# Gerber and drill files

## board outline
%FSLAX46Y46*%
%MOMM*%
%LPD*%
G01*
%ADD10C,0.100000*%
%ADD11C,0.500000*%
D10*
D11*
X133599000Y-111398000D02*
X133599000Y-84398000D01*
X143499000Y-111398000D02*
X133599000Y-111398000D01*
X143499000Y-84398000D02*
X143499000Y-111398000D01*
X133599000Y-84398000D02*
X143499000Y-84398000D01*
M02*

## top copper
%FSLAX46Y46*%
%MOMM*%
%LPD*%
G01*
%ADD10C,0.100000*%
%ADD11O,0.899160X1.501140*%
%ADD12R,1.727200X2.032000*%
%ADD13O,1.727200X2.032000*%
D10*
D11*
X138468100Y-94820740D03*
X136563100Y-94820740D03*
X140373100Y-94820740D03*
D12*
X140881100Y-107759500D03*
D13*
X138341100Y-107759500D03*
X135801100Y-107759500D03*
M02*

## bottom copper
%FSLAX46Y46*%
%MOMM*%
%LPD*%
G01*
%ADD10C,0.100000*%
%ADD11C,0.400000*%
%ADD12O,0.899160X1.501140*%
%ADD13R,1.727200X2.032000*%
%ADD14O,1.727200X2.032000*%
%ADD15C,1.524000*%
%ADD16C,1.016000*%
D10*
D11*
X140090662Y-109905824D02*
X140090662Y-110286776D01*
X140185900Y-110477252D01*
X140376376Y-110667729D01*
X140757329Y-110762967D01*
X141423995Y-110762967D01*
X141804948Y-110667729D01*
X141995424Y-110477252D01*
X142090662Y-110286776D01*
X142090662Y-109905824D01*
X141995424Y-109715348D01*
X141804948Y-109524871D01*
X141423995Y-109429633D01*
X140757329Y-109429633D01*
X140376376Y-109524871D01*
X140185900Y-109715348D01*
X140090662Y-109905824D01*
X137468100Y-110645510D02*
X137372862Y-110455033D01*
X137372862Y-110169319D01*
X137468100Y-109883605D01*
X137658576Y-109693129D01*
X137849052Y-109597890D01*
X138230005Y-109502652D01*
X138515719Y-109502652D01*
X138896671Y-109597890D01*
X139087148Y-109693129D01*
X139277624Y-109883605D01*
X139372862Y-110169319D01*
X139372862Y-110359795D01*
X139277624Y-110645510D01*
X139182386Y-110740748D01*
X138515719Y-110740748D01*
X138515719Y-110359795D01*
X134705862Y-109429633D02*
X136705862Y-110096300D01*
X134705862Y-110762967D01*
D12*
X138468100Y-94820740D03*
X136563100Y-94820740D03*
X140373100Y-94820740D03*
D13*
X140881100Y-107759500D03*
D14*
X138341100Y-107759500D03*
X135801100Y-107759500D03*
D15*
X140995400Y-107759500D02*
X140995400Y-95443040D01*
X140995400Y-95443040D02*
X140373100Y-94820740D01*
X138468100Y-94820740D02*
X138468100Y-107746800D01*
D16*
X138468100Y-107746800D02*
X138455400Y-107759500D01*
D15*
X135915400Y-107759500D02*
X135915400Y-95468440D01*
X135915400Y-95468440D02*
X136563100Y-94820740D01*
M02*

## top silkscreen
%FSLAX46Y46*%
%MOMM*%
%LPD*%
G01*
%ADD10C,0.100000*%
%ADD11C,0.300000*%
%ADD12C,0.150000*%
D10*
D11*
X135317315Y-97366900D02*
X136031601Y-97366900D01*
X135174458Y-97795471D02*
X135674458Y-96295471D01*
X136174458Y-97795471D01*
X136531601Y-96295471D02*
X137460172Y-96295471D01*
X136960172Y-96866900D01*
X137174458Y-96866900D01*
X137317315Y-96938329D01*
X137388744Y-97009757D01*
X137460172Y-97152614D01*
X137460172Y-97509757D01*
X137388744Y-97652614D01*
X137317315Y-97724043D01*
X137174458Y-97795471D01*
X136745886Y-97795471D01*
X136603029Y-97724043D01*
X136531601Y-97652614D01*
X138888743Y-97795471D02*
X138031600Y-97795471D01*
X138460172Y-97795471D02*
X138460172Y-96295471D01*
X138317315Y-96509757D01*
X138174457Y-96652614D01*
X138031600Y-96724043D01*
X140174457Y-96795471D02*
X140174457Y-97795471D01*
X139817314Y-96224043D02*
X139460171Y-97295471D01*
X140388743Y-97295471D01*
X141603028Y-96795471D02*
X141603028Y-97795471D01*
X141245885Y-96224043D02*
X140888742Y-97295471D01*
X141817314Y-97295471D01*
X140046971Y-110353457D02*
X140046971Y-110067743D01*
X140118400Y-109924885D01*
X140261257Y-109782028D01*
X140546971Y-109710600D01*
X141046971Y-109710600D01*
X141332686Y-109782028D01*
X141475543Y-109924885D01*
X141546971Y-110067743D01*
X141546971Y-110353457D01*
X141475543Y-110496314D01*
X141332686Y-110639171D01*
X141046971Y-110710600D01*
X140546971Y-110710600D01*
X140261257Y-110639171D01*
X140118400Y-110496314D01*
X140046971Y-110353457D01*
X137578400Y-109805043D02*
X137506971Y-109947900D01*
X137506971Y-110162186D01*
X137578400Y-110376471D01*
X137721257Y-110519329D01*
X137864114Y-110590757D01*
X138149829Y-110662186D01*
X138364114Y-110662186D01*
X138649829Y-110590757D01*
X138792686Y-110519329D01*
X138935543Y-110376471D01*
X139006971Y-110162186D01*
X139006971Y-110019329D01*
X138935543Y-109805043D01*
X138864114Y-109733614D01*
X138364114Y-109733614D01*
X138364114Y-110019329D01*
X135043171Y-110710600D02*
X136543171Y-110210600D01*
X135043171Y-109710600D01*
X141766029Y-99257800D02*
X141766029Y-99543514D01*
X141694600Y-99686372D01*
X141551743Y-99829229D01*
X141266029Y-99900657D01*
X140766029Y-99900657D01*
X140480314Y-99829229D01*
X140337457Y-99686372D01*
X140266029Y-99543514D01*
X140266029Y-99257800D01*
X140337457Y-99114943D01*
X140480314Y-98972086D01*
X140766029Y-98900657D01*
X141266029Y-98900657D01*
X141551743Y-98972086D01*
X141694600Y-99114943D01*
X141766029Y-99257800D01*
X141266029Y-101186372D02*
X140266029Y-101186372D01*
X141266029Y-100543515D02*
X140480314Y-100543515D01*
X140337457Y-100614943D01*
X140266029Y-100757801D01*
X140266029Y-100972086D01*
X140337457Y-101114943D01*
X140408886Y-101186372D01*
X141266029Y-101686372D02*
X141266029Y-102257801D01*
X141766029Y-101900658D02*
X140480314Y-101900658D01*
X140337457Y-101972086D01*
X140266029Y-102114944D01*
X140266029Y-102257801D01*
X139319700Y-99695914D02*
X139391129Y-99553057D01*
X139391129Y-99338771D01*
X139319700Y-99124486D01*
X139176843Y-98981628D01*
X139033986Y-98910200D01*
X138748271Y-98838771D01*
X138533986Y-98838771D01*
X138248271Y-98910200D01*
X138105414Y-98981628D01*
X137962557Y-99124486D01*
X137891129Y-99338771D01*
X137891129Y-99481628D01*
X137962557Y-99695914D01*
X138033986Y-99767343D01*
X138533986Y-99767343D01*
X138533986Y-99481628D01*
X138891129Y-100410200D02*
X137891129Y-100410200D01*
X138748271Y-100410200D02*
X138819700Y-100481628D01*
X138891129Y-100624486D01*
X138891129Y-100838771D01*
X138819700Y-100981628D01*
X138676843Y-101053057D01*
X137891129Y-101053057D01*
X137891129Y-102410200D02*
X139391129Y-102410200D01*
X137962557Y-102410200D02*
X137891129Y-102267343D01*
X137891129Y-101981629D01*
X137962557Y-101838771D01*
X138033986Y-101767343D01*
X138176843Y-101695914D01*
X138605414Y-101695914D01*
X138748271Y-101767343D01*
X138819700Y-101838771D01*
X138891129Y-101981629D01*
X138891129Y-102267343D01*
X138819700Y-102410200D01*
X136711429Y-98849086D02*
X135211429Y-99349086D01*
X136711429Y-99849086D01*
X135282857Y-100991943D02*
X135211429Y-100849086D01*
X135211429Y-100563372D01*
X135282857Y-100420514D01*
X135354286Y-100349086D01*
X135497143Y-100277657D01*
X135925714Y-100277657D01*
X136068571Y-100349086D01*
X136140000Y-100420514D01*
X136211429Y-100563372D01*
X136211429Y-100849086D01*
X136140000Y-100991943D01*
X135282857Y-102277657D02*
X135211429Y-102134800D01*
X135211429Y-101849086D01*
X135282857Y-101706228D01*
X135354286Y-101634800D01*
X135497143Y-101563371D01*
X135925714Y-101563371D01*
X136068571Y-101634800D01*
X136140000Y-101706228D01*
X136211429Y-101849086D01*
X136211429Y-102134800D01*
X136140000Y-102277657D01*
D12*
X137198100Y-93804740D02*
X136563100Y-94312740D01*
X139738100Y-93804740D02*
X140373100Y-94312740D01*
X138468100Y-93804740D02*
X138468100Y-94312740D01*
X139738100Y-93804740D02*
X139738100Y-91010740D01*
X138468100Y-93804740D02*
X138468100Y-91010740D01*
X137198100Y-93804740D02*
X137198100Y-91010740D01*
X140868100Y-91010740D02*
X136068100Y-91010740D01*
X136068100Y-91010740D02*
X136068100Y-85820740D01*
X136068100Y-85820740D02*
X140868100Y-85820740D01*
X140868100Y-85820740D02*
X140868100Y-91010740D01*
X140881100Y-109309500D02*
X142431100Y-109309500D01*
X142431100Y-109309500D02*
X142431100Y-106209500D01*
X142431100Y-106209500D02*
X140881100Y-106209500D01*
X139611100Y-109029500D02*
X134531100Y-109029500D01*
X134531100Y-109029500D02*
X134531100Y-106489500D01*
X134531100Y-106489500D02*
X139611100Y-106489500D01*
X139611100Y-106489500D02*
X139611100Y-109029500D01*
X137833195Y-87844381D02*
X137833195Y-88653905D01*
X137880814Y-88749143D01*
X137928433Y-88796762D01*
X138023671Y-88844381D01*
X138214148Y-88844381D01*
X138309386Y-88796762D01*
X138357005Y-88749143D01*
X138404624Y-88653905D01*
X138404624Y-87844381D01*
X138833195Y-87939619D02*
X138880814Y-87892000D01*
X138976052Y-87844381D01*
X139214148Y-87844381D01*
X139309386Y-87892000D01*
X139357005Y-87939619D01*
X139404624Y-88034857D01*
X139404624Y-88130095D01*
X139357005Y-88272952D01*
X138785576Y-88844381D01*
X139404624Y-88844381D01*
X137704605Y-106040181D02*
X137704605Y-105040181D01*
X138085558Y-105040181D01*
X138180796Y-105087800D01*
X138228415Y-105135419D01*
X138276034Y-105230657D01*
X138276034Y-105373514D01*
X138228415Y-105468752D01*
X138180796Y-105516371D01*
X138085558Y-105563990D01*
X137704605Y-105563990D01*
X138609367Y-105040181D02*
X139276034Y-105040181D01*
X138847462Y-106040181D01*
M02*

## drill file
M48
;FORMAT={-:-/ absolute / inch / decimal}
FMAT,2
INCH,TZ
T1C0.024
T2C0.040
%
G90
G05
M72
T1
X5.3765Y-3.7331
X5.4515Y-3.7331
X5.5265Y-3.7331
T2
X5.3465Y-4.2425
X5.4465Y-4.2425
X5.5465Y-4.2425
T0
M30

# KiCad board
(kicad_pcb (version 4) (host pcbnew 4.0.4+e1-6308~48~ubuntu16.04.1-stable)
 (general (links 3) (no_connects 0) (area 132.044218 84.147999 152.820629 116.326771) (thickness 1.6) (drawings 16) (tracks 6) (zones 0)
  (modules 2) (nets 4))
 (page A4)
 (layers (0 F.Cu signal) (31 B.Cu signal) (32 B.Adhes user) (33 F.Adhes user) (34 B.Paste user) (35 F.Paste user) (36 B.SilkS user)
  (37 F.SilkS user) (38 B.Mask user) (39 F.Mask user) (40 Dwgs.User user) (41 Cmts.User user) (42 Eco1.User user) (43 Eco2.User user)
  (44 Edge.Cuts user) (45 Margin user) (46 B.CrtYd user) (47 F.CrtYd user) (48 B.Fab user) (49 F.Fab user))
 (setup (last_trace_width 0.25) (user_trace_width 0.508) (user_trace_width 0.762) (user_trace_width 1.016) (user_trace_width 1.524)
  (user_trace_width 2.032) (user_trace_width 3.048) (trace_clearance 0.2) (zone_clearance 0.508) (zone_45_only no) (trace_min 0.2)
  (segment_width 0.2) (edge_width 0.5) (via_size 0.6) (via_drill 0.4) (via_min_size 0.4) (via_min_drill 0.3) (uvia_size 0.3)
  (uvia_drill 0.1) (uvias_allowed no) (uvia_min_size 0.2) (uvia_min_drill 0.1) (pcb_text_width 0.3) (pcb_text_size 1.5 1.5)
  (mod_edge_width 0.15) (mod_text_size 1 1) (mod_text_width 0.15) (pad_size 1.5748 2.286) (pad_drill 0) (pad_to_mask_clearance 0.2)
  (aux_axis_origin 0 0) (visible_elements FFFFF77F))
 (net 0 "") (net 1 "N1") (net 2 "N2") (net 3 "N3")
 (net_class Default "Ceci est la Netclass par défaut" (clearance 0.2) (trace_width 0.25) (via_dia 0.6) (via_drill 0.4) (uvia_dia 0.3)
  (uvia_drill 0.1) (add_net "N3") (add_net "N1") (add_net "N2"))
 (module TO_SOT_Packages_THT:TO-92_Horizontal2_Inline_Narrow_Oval (layer F.Cu) (at 137.1981 94.82074)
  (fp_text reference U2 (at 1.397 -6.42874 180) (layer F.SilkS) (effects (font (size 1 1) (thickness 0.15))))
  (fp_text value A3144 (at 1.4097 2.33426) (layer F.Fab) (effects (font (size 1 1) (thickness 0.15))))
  (fp_line (start 0 -1.016) (end -0.635 -0.508) (layer F.SilkS) (width 0.15))
  (fp_line (start 2.54 -1.016) (end 3.175 -0.508) (layer F.SilkS) (width 0.15))
  (fp_line (start 1.27 -1.016) (end 1.27 -0.508) (layer F.SilkS) (width 0.15))
  (fp_line (start 2.54 -1.016) (end 2.54 -3.81) (layer F.SilkS) (width 0.15))
  (fp_line (start 1.27 -1.016) (end 1.27 -3.81) (layer F.SilkS) (width 0.15))
  (fp_line (start 0 -1.016) (end 0 -3.81) (layer F.SilkS) (width 0.15))
  (fp_line (start 3.67 -3.81) (end -1.13 -3.81) (layer F.SilkS) (width 0.15))
  (fp_line (start -1.13 -3.81) (end -1.13 -9) (layer F.SilkS) (width 0.15))
  (fp_line (start -1.13 -9) (end 3.67 -9) (layer F.SilkS) (width 0.15))
  (fp_line (start 3.67 -9) (end 3.67 -3.81) (layer F.SilkS) (width 0.15))
  (pad 2 thru_hole oval (at 1.27 0) (size 0.89916 1.50114) (drill 0.6) (layers *.Cu *.Mask F.SilkS) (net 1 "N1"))
  (pad 1 thru_hole oval (at -0.635 0) (size 0.89916 1.50114) (drill 0.6) (layers *.Cu *.Mask F.SilkS) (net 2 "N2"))
  (pad 3 thru_hole oval (at 3.175 0) (size 0.89916 1.50114) (drill 0.6) (layers *.Cu *.Mask F.SilkS) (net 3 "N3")))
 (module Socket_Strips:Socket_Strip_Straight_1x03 (layer F.Cu) (at 140.8811 107.7595 180)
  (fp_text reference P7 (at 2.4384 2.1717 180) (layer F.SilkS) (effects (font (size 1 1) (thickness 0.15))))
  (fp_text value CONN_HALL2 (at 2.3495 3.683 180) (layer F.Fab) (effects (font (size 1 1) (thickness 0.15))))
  (fp_line (start 0 -1.55) (end -1.55 -1.55) (layer F.SilkS) (width 0.15))
  (fp_line (start -1.55 -1.55) (end -1.55 1.55) (layer F.SilkS) (width 0.15))
  (fp_line (start -1.55 1.55) (end 0 1.55) (layer F.SilkS) (width 0.15))
  (fp_line (start 1.27 -1.27) (end 6.35 -1.27) (layer F.SilkS) (width 0.15))
  (fp_line (start 6.35 -1.27) (end 6.35 1.27) (layer F.SilkS) (width 0.15))
  (fp_line (start 6.35 1.27) (end 1.27 1.27) (layer F.SilkS) (width 0.15))
  (fp_line (start 1.27 1.27) (end 1.27 -1.27) (layer F.SilkS) (width 0.15))
  (pad 1 thru_hole rect (at 0 0 180) (size 1.7272 2.032) (drill 1.016) (layers *.Cu *.Mask F.SilkS) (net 3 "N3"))
  (pad 2 thru_hole oval (at 2.54 0 180) (size 1.7272 2.032) (drill 1.016) (layers *.Cu *.Mask F.SilkS) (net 1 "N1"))
  (pad 3 thru_hole oval (at 5.08 0 180) (size 1.7272 2.032) (drill 1.016) (layers *.Cu *.Mask F.SilkS) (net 2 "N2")))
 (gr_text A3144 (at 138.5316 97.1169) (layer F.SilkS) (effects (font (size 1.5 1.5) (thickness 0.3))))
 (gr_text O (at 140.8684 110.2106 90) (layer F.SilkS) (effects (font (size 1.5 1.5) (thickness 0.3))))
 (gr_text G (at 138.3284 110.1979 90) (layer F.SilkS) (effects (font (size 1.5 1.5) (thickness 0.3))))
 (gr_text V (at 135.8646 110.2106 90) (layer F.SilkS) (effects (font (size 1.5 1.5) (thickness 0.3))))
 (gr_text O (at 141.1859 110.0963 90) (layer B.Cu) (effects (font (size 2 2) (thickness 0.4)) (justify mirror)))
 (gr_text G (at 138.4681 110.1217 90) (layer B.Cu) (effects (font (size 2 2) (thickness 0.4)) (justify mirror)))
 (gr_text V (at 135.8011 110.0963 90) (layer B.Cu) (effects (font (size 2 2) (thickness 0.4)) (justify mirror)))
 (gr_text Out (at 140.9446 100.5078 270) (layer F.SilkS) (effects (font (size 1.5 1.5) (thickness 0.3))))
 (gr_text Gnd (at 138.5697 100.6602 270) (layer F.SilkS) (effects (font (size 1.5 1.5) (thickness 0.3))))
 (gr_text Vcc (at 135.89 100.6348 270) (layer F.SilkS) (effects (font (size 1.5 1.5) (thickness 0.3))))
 (gr_line (start 133.599 111.398) (end 133.599 84.398) (angle 90) (layer Edge.Cuts) (width 0.5))
 (gr_line (start 143.499 111.398) (end 133.599 111.398) (angle 90) (layer Edge.Cuts) (width 0.5))
 (gr_line (start 143.499 84.398) (end 143.499 111.398) (angle 90) (layer Edge.Cuts) (width 0.5))
 (gr_line (start 133.599 84.398) (end 143.499 84.398) (angle 90) (layer Edge.Cuts) (width 0.5))
 (segment (start 140.9954 107.7595) (end 140.9954 95.44304) (width 1.524) (layer B.Cu) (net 3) (status 10))
 (segment (start 140.9954 95.44304) (end 140.3731 94.82074) (width 1.524) (layer B.Cu) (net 3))
 (segment (start 138.4681 94.82074) (end 138.4681 107.7468) (width 1.524) (layer B.Cu) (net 1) (status 20))
 (segment (start 138.4681 107.7468) (end 138.4554 107.7595) (width 1.016) (layer B.Cu) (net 1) (status 30))
 (segment (start 135.9154 107.7595) (end 135.9154 95.46844) (width 1.524) (layer B.Cu) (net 2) (status 10))
 (segment (start 135.9154 95.46844) (end 136.5631 94.82074) (width 1.524) (layer B.Cu) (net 2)))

